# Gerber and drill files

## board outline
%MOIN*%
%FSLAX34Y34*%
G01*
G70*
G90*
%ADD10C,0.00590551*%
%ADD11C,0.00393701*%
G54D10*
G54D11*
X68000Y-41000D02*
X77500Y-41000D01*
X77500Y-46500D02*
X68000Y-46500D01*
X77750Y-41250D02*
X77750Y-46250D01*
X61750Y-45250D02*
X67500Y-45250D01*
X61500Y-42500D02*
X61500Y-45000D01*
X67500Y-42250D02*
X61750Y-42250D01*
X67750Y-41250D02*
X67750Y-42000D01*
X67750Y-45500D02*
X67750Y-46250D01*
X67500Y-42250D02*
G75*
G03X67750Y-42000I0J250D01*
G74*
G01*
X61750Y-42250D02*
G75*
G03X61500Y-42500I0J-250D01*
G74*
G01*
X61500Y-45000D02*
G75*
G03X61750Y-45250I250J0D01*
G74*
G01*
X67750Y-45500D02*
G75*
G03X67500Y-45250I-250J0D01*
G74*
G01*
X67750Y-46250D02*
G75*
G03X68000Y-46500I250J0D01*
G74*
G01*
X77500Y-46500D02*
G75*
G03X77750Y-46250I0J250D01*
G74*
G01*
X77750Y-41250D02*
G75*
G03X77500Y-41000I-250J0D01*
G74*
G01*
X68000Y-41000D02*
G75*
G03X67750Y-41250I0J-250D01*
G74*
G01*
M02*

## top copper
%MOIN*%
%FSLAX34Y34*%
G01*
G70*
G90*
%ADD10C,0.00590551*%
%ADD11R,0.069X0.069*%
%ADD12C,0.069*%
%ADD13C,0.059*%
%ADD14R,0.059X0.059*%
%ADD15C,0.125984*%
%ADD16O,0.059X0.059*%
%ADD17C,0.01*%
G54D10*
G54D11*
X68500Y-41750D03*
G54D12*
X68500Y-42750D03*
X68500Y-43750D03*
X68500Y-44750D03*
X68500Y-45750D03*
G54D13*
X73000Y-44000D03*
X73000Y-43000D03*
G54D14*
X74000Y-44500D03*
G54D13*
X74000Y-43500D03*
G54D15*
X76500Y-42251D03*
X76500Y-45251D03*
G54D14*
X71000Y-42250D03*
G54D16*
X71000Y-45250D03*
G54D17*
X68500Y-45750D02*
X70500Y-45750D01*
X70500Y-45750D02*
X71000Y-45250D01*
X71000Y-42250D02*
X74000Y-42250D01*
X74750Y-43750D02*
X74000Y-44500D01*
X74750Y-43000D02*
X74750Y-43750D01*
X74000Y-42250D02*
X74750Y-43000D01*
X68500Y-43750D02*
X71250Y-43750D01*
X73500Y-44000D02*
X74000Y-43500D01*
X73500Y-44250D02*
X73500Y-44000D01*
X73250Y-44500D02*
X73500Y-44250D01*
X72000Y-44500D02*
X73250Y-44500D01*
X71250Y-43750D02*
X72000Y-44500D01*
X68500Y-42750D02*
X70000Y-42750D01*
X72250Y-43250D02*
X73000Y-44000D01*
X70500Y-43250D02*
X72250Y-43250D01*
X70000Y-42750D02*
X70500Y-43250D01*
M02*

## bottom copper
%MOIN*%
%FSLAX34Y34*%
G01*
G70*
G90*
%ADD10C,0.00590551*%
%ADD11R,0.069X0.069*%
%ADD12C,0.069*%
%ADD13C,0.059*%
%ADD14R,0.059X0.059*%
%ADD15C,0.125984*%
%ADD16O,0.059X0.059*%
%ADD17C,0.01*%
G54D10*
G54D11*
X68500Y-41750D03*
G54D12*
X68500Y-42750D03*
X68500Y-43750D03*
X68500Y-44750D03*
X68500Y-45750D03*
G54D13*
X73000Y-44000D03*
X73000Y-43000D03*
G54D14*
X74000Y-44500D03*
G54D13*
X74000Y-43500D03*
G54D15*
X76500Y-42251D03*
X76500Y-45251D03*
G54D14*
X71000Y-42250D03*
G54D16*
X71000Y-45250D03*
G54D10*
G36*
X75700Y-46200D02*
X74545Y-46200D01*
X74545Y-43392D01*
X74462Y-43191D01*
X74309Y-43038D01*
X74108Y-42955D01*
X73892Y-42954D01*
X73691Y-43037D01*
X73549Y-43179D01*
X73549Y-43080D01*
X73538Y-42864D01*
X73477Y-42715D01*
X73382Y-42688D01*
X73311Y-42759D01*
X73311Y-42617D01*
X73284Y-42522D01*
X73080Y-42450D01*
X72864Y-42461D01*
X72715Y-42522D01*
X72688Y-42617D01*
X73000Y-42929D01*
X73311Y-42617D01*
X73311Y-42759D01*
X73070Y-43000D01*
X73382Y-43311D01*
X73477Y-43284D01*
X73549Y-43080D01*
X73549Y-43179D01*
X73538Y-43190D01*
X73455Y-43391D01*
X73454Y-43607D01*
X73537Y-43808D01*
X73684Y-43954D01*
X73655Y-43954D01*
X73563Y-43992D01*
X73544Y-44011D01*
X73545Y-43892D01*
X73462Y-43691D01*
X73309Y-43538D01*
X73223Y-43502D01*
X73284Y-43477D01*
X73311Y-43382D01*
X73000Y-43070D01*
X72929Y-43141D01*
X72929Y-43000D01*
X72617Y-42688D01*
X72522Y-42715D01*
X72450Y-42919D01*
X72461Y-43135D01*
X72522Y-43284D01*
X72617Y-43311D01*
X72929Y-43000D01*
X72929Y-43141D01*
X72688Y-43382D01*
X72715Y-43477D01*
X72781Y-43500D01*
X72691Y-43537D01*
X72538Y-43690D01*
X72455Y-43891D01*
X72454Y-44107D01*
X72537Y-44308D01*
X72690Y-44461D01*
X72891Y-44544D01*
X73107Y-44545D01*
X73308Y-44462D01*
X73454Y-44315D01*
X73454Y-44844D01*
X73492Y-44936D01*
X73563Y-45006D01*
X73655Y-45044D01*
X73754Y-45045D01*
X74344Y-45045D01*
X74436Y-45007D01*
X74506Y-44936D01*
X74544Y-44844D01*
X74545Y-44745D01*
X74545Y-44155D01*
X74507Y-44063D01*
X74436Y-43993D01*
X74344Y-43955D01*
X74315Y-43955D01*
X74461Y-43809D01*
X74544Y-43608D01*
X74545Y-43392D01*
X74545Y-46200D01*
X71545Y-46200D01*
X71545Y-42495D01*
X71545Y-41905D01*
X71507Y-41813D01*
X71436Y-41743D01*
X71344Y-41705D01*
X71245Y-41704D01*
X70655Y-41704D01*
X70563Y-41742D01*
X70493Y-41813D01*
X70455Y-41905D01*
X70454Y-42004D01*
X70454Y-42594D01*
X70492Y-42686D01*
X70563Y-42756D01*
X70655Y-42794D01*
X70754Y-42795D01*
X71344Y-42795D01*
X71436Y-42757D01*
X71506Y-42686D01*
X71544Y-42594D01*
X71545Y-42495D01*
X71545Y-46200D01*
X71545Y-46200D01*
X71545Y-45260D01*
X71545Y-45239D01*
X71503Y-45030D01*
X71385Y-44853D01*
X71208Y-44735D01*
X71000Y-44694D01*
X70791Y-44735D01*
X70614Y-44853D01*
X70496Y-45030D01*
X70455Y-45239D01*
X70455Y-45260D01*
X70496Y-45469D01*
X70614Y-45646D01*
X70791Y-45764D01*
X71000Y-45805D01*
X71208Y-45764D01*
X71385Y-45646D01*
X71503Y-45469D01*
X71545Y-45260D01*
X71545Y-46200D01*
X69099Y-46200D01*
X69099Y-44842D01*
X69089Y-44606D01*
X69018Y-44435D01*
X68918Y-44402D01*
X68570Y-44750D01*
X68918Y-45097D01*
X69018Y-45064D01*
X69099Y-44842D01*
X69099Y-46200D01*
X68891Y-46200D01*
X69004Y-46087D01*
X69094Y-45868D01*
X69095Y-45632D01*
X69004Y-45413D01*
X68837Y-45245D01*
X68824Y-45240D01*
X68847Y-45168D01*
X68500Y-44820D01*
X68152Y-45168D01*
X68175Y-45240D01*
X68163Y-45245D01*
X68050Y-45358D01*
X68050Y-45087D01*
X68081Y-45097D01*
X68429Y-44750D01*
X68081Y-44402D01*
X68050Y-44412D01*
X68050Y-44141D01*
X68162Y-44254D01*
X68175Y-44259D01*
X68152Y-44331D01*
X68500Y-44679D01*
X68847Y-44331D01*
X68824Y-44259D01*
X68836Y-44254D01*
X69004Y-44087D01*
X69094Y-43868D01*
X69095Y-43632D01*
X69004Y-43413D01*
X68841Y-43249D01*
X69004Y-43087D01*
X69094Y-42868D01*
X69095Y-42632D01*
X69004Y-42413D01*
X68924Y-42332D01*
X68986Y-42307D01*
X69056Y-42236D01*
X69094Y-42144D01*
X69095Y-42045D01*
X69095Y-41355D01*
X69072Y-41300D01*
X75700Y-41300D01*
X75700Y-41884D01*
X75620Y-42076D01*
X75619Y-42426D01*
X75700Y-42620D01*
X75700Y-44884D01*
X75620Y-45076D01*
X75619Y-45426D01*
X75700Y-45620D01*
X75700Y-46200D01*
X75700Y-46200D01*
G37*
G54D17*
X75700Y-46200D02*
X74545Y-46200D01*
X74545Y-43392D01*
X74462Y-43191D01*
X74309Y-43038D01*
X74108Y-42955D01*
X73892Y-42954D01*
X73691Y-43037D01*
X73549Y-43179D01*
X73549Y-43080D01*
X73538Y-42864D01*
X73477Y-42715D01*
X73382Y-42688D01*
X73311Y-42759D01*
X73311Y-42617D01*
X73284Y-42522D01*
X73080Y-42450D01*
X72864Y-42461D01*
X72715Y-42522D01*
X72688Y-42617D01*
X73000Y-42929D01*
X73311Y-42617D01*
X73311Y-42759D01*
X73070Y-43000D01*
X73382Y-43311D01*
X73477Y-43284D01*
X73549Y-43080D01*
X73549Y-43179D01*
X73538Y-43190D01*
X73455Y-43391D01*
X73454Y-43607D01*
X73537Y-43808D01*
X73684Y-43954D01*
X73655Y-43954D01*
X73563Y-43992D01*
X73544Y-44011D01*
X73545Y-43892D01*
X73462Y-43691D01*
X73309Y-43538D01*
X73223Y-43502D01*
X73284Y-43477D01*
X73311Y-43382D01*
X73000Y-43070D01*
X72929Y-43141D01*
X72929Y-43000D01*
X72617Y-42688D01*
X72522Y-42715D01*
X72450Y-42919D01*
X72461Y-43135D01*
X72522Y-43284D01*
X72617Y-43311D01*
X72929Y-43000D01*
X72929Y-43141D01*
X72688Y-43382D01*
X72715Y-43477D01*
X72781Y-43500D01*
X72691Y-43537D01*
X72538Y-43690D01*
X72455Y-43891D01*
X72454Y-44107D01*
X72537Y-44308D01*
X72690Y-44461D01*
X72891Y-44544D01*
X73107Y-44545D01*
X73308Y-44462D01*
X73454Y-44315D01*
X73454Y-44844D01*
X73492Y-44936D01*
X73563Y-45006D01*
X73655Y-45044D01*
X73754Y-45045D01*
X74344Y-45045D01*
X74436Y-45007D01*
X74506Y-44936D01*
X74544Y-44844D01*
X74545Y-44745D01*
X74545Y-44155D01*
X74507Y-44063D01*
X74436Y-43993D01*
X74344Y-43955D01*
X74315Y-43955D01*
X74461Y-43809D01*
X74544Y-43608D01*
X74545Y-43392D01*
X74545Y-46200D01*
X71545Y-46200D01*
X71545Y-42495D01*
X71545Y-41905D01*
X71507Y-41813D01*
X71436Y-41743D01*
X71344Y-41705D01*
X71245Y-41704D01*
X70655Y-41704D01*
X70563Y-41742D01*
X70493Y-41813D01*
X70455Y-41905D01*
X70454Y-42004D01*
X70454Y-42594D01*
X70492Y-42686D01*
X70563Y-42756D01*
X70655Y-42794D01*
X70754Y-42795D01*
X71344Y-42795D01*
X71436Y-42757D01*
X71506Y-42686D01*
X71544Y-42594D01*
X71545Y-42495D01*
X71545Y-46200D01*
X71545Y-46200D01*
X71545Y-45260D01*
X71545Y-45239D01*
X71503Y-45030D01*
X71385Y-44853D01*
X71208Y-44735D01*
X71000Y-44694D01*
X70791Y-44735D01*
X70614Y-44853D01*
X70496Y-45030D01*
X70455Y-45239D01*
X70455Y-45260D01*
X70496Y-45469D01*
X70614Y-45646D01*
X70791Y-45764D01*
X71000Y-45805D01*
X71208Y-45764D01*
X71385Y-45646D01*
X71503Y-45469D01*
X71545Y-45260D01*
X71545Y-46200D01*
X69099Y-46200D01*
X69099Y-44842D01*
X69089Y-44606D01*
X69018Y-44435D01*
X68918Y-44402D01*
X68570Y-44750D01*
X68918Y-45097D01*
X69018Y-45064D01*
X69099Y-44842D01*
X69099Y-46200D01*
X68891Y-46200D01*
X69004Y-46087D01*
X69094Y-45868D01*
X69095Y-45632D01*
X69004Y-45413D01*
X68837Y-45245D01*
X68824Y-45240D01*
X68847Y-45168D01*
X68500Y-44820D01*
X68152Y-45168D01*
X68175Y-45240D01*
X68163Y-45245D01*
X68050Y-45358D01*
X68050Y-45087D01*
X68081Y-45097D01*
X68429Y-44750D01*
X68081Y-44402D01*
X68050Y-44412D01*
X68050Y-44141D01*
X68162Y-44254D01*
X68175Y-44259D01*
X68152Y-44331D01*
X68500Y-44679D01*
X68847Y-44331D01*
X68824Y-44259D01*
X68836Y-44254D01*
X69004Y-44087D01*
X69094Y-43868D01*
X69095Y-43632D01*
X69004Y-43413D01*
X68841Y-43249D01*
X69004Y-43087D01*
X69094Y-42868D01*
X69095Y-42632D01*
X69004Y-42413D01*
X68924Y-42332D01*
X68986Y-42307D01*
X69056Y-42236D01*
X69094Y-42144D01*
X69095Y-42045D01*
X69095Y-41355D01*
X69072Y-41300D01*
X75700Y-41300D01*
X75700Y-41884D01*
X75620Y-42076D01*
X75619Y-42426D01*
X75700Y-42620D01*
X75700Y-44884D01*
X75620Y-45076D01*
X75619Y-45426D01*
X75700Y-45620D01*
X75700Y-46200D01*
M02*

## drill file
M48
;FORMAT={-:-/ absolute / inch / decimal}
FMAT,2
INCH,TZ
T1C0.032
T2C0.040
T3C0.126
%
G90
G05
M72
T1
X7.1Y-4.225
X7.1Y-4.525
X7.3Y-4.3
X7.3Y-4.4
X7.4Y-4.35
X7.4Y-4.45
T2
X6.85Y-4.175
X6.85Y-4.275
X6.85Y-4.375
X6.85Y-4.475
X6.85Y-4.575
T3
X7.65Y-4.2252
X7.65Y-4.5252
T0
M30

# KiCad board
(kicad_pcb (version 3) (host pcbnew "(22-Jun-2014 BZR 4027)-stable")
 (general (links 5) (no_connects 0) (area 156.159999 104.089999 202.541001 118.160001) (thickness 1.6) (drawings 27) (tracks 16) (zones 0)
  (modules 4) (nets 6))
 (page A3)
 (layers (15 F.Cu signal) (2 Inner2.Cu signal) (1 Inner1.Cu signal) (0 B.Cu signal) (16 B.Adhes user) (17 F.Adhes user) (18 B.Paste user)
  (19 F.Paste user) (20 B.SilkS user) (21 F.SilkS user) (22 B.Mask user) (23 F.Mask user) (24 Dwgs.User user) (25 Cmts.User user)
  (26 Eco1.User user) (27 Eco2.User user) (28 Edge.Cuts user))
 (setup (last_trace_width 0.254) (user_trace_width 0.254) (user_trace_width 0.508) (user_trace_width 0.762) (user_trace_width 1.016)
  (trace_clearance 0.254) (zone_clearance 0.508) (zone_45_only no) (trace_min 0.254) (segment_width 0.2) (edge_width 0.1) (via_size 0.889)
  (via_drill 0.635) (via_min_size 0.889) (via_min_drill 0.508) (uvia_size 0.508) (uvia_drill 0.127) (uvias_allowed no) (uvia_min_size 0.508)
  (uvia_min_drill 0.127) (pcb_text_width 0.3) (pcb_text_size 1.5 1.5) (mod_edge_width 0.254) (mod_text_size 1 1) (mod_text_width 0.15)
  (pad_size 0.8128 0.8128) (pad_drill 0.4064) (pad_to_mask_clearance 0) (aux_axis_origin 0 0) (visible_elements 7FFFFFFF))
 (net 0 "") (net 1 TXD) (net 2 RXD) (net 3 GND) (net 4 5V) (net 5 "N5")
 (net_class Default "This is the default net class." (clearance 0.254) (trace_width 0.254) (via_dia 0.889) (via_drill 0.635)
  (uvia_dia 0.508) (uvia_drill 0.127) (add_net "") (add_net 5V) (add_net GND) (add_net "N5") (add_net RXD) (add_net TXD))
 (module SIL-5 (layer F.Cu) (at 173.99 108.585 270)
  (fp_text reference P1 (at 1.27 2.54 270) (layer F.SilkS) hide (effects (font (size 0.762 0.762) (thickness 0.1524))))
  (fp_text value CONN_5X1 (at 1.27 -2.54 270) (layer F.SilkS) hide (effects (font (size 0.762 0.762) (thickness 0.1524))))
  (pad 1 thru_hole rect (at -2.54 0 270) (size 1.7526 1.7526) (drill 1.016) (layers *.Cu *.Mask F.SilkS))
  (pad 2 thru_hole circle (at 0 0 270) (size 1.7526 1.7526) (drill 1.016) (layers *.Cu *.Mask F.SilkS) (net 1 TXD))
  (pad 3 thru_hole circle (at 2.54 0 270) (size 1.7526 1.7526) (drill 1.016) (layers *.Cu *.Mask F.SilkS) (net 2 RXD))
  (pad 4 thru_hole circle (at 5.08 0 270) (size 1.7526 1.7526) (drill 1.016) (layers *.Cu *.Mask F.SilkS) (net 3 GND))
  (pad 5 thru_hole circle (at 7.62 0 270) (size 1.7526 1.7526) (drill 1.016) (layers *.Cu *.Mask F.SilkS) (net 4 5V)))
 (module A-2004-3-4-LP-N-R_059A (layer F.Cu) (at 187.96 113.03 90)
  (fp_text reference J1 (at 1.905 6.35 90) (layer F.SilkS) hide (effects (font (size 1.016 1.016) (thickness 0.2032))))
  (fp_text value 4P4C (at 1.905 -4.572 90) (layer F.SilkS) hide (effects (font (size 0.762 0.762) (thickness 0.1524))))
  (pad 2 thru_hole circle (at 1.27 -2.54 90) (size 1.4986 1.4986) (drill 0.8128) (layers *.Cu *.Mask F.SilkS) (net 1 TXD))
  (pad 4 thru_hole circle (at 3.81 -2.54 90) (size 1.4986 1.4986) (drill 0.8128) (layers *.Cu *.Mask F.SilkS) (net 3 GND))
  (pad 1 thru_hole rect (at 0 0 90) (size 1.4986 1.4986) (drill 0.8128) (layers *.Cu *.Mask F.SilkS) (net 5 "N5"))
  (pad 3 thru_hole circle (at 2.54 0 90) (size 1.4986 1.4986) (drill 0.8128) (layers *.Cu *.Mask F.SilkS) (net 2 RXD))
  (pad "" thru_hole circle (at 5.71 6.35 90) (size 3.2 3.2) (drill 3.2) (layers *.Cu *.Mask F.SilkS))
  (pad "" thru_hole circle (at -1.91 6.35 90) (size 3.2 3.2) (drill 3.2) (layers *.Cu *.Mask F.SilkS)))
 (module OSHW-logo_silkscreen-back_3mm (layer F.Cu) (at 169.545 111.125)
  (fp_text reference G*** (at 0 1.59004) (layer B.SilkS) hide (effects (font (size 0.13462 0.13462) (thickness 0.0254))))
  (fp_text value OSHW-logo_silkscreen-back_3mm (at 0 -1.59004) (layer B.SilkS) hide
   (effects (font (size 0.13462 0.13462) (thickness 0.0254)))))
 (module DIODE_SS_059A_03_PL (layer F.Cu) (at 180.34 111.125 90)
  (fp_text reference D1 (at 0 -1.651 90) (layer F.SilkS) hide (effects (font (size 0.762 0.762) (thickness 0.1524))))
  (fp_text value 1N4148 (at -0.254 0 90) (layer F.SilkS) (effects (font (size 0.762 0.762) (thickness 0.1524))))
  (pad 2 thru_hole rect (at 3.81 0 90) (size 1.4986 1.4986) (drill 0.8128) (layers *.Cu *.Mask F.SilkS) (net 5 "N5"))
  (pad 1 thru_hole oval (at -3.81 0 90) (size 1.4986 1.4986) (drill 0.8128) (layers *.Cu *.Mask F.SilkS) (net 4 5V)))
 (gr_line (start 172.72 104.14) (end 196.85 104.14) (angle 90) (layer Edge.Cuts) (width 0.1))
 (gr_line (start 196.85 118.11) (end 172.72 118.11) (angle 90) (layer Edge.Cuts) (width 0.1))
 (gr_line (start 197.485 104.775) (end 197.485 117.475) (angle 90) (layer Edge.Cuts) (width 0.1))
 (gr_line (start 156.845 114.935) (end 171.45 114.935) (angle 90) (layer Edge.Cuts) (width 0.1))
 (gr_line (start 156.21 107.95) (end 156.21 114.3) (angle 90) (layer Edge.Cuts) (width 0.1))
 (gr_line (start 171.45 107.315) (end 156.845 107.315) (angle 90) (layer Edge.Cuts) (width 0.1))
 (gr_line (start 172.085 104.775) (end 172.085 106.68) (angle 90) (layer Edge.Cuts) (width 0.1))
 (gr_line (start 172.085 115.57) (end 172.085 117.475) (angle 90) (layer Edge.Cuts) (width 0.1))
 (gr_arc (start 171.45 106.68) (end 172.085 106.68) (angle 90) (layer Edge.Cuts) (width 0.1))
 (gr_arc (start 156.845 107.95) (end 156.21 107.95) (angle 90) (layer Edge.Cuts) (width 0.1))
 (gr_arc (start 156.845 114.3) (end 156.845 114.935) (angle 90) (layer Edge.Cuts) (width 0.1))
 (gr_arc (start 171.45 115.57) (end 171.45 114.935) (angle 90) (layer Edge.Cuts) (width 0.1))
 (gr_arc (start 172.72 117.475) (end 172.72 118.11) (angle 90) (layer Edge.Cuts) (width 0.1))
 (gr_arc (start 196.85 117.475) (end 197.485 117.475) (angle 90) (layer Edge.Cuts) (width 0.1))
 (gr_arc (start 196.85 104.775) (end 196.85 104.14) (angle 90) (layer Edge.Cuts) (width 0.1))
 (gr_arc (start 172.72 104.775) (end 172.085 104.775) (angle 90) (layer Edge.Cuts) (width 0.1))
 (segment (start 173.99 116.205) (end 179.07 116.205) (width 0.254) (layer F.Cu) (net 4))
 (segment (start 179.07 116.205) (end 180.34 114.935) (width 0.254) (layer F.Cu) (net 4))
 (segment (start 180.34 107.315) (end 187.96 107.315) (width 0.254) (layer F.Cu) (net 5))
 (segment (start 189.865 111.125) (end 187.96 113.03) (width 0.254) (layer F.Cu) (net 5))
 (segment (start 189.865 109.22) (end 189.865 111.125) (width 0.254) (layer F.Cu) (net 5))
 (segment (start 187.96 107.315) (end 189.865 109.22) (width 0.254) (layer F.Cu) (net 5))
 (segment (start 173.99 111.125) (end 180.975 111.125) (width 0.254) (layer F.Cu) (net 2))
 (segment (start 186.69 111.76) (end 187.96 110.49) (width 0.254) (layer F.Cu) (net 2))
 (segment (start 186.69 112.395) (end 186.69 111.76) (width 0.254) (layer F.Cu) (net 2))
 (segment (start 186.055 113.03) (end 186.69 112.395) (width 0.254) (layer F.Cu) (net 2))
 (segment (start 182.88 113.03) (end 186.055 113.03) (width 0.254) (layer F.Cu) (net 2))
 (segment (start 180.975 111.125) (end 182.88 113.03) (width 0.254) (layer F.Cu) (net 2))
 (segment (start 173.99 108.585) (end 177.8 108.585) (width 0.254) (layer F.Cu) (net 1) (status 400000))
 (segment (start 183.515 109.855) (end 185.42 111.76) (width 0.254) (layer F.Cu) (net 1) (status 800000))
 (segment (start 179.07 109.855) (end 183.515 109.855) (width 0.254) (layer F.Cu) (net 1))
 (segment (start 177.8 108.585) (end 179.07 109.855) (width 0.254) (layer F.Cu) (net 1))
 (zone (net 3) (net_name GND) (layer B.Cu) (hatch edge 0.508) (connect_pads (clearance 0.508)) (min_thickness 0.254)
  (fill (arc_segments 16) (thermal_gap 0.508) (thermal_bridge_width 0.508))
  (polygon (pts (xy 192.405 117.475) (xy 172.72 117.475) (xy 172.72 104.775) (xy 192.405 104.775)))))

